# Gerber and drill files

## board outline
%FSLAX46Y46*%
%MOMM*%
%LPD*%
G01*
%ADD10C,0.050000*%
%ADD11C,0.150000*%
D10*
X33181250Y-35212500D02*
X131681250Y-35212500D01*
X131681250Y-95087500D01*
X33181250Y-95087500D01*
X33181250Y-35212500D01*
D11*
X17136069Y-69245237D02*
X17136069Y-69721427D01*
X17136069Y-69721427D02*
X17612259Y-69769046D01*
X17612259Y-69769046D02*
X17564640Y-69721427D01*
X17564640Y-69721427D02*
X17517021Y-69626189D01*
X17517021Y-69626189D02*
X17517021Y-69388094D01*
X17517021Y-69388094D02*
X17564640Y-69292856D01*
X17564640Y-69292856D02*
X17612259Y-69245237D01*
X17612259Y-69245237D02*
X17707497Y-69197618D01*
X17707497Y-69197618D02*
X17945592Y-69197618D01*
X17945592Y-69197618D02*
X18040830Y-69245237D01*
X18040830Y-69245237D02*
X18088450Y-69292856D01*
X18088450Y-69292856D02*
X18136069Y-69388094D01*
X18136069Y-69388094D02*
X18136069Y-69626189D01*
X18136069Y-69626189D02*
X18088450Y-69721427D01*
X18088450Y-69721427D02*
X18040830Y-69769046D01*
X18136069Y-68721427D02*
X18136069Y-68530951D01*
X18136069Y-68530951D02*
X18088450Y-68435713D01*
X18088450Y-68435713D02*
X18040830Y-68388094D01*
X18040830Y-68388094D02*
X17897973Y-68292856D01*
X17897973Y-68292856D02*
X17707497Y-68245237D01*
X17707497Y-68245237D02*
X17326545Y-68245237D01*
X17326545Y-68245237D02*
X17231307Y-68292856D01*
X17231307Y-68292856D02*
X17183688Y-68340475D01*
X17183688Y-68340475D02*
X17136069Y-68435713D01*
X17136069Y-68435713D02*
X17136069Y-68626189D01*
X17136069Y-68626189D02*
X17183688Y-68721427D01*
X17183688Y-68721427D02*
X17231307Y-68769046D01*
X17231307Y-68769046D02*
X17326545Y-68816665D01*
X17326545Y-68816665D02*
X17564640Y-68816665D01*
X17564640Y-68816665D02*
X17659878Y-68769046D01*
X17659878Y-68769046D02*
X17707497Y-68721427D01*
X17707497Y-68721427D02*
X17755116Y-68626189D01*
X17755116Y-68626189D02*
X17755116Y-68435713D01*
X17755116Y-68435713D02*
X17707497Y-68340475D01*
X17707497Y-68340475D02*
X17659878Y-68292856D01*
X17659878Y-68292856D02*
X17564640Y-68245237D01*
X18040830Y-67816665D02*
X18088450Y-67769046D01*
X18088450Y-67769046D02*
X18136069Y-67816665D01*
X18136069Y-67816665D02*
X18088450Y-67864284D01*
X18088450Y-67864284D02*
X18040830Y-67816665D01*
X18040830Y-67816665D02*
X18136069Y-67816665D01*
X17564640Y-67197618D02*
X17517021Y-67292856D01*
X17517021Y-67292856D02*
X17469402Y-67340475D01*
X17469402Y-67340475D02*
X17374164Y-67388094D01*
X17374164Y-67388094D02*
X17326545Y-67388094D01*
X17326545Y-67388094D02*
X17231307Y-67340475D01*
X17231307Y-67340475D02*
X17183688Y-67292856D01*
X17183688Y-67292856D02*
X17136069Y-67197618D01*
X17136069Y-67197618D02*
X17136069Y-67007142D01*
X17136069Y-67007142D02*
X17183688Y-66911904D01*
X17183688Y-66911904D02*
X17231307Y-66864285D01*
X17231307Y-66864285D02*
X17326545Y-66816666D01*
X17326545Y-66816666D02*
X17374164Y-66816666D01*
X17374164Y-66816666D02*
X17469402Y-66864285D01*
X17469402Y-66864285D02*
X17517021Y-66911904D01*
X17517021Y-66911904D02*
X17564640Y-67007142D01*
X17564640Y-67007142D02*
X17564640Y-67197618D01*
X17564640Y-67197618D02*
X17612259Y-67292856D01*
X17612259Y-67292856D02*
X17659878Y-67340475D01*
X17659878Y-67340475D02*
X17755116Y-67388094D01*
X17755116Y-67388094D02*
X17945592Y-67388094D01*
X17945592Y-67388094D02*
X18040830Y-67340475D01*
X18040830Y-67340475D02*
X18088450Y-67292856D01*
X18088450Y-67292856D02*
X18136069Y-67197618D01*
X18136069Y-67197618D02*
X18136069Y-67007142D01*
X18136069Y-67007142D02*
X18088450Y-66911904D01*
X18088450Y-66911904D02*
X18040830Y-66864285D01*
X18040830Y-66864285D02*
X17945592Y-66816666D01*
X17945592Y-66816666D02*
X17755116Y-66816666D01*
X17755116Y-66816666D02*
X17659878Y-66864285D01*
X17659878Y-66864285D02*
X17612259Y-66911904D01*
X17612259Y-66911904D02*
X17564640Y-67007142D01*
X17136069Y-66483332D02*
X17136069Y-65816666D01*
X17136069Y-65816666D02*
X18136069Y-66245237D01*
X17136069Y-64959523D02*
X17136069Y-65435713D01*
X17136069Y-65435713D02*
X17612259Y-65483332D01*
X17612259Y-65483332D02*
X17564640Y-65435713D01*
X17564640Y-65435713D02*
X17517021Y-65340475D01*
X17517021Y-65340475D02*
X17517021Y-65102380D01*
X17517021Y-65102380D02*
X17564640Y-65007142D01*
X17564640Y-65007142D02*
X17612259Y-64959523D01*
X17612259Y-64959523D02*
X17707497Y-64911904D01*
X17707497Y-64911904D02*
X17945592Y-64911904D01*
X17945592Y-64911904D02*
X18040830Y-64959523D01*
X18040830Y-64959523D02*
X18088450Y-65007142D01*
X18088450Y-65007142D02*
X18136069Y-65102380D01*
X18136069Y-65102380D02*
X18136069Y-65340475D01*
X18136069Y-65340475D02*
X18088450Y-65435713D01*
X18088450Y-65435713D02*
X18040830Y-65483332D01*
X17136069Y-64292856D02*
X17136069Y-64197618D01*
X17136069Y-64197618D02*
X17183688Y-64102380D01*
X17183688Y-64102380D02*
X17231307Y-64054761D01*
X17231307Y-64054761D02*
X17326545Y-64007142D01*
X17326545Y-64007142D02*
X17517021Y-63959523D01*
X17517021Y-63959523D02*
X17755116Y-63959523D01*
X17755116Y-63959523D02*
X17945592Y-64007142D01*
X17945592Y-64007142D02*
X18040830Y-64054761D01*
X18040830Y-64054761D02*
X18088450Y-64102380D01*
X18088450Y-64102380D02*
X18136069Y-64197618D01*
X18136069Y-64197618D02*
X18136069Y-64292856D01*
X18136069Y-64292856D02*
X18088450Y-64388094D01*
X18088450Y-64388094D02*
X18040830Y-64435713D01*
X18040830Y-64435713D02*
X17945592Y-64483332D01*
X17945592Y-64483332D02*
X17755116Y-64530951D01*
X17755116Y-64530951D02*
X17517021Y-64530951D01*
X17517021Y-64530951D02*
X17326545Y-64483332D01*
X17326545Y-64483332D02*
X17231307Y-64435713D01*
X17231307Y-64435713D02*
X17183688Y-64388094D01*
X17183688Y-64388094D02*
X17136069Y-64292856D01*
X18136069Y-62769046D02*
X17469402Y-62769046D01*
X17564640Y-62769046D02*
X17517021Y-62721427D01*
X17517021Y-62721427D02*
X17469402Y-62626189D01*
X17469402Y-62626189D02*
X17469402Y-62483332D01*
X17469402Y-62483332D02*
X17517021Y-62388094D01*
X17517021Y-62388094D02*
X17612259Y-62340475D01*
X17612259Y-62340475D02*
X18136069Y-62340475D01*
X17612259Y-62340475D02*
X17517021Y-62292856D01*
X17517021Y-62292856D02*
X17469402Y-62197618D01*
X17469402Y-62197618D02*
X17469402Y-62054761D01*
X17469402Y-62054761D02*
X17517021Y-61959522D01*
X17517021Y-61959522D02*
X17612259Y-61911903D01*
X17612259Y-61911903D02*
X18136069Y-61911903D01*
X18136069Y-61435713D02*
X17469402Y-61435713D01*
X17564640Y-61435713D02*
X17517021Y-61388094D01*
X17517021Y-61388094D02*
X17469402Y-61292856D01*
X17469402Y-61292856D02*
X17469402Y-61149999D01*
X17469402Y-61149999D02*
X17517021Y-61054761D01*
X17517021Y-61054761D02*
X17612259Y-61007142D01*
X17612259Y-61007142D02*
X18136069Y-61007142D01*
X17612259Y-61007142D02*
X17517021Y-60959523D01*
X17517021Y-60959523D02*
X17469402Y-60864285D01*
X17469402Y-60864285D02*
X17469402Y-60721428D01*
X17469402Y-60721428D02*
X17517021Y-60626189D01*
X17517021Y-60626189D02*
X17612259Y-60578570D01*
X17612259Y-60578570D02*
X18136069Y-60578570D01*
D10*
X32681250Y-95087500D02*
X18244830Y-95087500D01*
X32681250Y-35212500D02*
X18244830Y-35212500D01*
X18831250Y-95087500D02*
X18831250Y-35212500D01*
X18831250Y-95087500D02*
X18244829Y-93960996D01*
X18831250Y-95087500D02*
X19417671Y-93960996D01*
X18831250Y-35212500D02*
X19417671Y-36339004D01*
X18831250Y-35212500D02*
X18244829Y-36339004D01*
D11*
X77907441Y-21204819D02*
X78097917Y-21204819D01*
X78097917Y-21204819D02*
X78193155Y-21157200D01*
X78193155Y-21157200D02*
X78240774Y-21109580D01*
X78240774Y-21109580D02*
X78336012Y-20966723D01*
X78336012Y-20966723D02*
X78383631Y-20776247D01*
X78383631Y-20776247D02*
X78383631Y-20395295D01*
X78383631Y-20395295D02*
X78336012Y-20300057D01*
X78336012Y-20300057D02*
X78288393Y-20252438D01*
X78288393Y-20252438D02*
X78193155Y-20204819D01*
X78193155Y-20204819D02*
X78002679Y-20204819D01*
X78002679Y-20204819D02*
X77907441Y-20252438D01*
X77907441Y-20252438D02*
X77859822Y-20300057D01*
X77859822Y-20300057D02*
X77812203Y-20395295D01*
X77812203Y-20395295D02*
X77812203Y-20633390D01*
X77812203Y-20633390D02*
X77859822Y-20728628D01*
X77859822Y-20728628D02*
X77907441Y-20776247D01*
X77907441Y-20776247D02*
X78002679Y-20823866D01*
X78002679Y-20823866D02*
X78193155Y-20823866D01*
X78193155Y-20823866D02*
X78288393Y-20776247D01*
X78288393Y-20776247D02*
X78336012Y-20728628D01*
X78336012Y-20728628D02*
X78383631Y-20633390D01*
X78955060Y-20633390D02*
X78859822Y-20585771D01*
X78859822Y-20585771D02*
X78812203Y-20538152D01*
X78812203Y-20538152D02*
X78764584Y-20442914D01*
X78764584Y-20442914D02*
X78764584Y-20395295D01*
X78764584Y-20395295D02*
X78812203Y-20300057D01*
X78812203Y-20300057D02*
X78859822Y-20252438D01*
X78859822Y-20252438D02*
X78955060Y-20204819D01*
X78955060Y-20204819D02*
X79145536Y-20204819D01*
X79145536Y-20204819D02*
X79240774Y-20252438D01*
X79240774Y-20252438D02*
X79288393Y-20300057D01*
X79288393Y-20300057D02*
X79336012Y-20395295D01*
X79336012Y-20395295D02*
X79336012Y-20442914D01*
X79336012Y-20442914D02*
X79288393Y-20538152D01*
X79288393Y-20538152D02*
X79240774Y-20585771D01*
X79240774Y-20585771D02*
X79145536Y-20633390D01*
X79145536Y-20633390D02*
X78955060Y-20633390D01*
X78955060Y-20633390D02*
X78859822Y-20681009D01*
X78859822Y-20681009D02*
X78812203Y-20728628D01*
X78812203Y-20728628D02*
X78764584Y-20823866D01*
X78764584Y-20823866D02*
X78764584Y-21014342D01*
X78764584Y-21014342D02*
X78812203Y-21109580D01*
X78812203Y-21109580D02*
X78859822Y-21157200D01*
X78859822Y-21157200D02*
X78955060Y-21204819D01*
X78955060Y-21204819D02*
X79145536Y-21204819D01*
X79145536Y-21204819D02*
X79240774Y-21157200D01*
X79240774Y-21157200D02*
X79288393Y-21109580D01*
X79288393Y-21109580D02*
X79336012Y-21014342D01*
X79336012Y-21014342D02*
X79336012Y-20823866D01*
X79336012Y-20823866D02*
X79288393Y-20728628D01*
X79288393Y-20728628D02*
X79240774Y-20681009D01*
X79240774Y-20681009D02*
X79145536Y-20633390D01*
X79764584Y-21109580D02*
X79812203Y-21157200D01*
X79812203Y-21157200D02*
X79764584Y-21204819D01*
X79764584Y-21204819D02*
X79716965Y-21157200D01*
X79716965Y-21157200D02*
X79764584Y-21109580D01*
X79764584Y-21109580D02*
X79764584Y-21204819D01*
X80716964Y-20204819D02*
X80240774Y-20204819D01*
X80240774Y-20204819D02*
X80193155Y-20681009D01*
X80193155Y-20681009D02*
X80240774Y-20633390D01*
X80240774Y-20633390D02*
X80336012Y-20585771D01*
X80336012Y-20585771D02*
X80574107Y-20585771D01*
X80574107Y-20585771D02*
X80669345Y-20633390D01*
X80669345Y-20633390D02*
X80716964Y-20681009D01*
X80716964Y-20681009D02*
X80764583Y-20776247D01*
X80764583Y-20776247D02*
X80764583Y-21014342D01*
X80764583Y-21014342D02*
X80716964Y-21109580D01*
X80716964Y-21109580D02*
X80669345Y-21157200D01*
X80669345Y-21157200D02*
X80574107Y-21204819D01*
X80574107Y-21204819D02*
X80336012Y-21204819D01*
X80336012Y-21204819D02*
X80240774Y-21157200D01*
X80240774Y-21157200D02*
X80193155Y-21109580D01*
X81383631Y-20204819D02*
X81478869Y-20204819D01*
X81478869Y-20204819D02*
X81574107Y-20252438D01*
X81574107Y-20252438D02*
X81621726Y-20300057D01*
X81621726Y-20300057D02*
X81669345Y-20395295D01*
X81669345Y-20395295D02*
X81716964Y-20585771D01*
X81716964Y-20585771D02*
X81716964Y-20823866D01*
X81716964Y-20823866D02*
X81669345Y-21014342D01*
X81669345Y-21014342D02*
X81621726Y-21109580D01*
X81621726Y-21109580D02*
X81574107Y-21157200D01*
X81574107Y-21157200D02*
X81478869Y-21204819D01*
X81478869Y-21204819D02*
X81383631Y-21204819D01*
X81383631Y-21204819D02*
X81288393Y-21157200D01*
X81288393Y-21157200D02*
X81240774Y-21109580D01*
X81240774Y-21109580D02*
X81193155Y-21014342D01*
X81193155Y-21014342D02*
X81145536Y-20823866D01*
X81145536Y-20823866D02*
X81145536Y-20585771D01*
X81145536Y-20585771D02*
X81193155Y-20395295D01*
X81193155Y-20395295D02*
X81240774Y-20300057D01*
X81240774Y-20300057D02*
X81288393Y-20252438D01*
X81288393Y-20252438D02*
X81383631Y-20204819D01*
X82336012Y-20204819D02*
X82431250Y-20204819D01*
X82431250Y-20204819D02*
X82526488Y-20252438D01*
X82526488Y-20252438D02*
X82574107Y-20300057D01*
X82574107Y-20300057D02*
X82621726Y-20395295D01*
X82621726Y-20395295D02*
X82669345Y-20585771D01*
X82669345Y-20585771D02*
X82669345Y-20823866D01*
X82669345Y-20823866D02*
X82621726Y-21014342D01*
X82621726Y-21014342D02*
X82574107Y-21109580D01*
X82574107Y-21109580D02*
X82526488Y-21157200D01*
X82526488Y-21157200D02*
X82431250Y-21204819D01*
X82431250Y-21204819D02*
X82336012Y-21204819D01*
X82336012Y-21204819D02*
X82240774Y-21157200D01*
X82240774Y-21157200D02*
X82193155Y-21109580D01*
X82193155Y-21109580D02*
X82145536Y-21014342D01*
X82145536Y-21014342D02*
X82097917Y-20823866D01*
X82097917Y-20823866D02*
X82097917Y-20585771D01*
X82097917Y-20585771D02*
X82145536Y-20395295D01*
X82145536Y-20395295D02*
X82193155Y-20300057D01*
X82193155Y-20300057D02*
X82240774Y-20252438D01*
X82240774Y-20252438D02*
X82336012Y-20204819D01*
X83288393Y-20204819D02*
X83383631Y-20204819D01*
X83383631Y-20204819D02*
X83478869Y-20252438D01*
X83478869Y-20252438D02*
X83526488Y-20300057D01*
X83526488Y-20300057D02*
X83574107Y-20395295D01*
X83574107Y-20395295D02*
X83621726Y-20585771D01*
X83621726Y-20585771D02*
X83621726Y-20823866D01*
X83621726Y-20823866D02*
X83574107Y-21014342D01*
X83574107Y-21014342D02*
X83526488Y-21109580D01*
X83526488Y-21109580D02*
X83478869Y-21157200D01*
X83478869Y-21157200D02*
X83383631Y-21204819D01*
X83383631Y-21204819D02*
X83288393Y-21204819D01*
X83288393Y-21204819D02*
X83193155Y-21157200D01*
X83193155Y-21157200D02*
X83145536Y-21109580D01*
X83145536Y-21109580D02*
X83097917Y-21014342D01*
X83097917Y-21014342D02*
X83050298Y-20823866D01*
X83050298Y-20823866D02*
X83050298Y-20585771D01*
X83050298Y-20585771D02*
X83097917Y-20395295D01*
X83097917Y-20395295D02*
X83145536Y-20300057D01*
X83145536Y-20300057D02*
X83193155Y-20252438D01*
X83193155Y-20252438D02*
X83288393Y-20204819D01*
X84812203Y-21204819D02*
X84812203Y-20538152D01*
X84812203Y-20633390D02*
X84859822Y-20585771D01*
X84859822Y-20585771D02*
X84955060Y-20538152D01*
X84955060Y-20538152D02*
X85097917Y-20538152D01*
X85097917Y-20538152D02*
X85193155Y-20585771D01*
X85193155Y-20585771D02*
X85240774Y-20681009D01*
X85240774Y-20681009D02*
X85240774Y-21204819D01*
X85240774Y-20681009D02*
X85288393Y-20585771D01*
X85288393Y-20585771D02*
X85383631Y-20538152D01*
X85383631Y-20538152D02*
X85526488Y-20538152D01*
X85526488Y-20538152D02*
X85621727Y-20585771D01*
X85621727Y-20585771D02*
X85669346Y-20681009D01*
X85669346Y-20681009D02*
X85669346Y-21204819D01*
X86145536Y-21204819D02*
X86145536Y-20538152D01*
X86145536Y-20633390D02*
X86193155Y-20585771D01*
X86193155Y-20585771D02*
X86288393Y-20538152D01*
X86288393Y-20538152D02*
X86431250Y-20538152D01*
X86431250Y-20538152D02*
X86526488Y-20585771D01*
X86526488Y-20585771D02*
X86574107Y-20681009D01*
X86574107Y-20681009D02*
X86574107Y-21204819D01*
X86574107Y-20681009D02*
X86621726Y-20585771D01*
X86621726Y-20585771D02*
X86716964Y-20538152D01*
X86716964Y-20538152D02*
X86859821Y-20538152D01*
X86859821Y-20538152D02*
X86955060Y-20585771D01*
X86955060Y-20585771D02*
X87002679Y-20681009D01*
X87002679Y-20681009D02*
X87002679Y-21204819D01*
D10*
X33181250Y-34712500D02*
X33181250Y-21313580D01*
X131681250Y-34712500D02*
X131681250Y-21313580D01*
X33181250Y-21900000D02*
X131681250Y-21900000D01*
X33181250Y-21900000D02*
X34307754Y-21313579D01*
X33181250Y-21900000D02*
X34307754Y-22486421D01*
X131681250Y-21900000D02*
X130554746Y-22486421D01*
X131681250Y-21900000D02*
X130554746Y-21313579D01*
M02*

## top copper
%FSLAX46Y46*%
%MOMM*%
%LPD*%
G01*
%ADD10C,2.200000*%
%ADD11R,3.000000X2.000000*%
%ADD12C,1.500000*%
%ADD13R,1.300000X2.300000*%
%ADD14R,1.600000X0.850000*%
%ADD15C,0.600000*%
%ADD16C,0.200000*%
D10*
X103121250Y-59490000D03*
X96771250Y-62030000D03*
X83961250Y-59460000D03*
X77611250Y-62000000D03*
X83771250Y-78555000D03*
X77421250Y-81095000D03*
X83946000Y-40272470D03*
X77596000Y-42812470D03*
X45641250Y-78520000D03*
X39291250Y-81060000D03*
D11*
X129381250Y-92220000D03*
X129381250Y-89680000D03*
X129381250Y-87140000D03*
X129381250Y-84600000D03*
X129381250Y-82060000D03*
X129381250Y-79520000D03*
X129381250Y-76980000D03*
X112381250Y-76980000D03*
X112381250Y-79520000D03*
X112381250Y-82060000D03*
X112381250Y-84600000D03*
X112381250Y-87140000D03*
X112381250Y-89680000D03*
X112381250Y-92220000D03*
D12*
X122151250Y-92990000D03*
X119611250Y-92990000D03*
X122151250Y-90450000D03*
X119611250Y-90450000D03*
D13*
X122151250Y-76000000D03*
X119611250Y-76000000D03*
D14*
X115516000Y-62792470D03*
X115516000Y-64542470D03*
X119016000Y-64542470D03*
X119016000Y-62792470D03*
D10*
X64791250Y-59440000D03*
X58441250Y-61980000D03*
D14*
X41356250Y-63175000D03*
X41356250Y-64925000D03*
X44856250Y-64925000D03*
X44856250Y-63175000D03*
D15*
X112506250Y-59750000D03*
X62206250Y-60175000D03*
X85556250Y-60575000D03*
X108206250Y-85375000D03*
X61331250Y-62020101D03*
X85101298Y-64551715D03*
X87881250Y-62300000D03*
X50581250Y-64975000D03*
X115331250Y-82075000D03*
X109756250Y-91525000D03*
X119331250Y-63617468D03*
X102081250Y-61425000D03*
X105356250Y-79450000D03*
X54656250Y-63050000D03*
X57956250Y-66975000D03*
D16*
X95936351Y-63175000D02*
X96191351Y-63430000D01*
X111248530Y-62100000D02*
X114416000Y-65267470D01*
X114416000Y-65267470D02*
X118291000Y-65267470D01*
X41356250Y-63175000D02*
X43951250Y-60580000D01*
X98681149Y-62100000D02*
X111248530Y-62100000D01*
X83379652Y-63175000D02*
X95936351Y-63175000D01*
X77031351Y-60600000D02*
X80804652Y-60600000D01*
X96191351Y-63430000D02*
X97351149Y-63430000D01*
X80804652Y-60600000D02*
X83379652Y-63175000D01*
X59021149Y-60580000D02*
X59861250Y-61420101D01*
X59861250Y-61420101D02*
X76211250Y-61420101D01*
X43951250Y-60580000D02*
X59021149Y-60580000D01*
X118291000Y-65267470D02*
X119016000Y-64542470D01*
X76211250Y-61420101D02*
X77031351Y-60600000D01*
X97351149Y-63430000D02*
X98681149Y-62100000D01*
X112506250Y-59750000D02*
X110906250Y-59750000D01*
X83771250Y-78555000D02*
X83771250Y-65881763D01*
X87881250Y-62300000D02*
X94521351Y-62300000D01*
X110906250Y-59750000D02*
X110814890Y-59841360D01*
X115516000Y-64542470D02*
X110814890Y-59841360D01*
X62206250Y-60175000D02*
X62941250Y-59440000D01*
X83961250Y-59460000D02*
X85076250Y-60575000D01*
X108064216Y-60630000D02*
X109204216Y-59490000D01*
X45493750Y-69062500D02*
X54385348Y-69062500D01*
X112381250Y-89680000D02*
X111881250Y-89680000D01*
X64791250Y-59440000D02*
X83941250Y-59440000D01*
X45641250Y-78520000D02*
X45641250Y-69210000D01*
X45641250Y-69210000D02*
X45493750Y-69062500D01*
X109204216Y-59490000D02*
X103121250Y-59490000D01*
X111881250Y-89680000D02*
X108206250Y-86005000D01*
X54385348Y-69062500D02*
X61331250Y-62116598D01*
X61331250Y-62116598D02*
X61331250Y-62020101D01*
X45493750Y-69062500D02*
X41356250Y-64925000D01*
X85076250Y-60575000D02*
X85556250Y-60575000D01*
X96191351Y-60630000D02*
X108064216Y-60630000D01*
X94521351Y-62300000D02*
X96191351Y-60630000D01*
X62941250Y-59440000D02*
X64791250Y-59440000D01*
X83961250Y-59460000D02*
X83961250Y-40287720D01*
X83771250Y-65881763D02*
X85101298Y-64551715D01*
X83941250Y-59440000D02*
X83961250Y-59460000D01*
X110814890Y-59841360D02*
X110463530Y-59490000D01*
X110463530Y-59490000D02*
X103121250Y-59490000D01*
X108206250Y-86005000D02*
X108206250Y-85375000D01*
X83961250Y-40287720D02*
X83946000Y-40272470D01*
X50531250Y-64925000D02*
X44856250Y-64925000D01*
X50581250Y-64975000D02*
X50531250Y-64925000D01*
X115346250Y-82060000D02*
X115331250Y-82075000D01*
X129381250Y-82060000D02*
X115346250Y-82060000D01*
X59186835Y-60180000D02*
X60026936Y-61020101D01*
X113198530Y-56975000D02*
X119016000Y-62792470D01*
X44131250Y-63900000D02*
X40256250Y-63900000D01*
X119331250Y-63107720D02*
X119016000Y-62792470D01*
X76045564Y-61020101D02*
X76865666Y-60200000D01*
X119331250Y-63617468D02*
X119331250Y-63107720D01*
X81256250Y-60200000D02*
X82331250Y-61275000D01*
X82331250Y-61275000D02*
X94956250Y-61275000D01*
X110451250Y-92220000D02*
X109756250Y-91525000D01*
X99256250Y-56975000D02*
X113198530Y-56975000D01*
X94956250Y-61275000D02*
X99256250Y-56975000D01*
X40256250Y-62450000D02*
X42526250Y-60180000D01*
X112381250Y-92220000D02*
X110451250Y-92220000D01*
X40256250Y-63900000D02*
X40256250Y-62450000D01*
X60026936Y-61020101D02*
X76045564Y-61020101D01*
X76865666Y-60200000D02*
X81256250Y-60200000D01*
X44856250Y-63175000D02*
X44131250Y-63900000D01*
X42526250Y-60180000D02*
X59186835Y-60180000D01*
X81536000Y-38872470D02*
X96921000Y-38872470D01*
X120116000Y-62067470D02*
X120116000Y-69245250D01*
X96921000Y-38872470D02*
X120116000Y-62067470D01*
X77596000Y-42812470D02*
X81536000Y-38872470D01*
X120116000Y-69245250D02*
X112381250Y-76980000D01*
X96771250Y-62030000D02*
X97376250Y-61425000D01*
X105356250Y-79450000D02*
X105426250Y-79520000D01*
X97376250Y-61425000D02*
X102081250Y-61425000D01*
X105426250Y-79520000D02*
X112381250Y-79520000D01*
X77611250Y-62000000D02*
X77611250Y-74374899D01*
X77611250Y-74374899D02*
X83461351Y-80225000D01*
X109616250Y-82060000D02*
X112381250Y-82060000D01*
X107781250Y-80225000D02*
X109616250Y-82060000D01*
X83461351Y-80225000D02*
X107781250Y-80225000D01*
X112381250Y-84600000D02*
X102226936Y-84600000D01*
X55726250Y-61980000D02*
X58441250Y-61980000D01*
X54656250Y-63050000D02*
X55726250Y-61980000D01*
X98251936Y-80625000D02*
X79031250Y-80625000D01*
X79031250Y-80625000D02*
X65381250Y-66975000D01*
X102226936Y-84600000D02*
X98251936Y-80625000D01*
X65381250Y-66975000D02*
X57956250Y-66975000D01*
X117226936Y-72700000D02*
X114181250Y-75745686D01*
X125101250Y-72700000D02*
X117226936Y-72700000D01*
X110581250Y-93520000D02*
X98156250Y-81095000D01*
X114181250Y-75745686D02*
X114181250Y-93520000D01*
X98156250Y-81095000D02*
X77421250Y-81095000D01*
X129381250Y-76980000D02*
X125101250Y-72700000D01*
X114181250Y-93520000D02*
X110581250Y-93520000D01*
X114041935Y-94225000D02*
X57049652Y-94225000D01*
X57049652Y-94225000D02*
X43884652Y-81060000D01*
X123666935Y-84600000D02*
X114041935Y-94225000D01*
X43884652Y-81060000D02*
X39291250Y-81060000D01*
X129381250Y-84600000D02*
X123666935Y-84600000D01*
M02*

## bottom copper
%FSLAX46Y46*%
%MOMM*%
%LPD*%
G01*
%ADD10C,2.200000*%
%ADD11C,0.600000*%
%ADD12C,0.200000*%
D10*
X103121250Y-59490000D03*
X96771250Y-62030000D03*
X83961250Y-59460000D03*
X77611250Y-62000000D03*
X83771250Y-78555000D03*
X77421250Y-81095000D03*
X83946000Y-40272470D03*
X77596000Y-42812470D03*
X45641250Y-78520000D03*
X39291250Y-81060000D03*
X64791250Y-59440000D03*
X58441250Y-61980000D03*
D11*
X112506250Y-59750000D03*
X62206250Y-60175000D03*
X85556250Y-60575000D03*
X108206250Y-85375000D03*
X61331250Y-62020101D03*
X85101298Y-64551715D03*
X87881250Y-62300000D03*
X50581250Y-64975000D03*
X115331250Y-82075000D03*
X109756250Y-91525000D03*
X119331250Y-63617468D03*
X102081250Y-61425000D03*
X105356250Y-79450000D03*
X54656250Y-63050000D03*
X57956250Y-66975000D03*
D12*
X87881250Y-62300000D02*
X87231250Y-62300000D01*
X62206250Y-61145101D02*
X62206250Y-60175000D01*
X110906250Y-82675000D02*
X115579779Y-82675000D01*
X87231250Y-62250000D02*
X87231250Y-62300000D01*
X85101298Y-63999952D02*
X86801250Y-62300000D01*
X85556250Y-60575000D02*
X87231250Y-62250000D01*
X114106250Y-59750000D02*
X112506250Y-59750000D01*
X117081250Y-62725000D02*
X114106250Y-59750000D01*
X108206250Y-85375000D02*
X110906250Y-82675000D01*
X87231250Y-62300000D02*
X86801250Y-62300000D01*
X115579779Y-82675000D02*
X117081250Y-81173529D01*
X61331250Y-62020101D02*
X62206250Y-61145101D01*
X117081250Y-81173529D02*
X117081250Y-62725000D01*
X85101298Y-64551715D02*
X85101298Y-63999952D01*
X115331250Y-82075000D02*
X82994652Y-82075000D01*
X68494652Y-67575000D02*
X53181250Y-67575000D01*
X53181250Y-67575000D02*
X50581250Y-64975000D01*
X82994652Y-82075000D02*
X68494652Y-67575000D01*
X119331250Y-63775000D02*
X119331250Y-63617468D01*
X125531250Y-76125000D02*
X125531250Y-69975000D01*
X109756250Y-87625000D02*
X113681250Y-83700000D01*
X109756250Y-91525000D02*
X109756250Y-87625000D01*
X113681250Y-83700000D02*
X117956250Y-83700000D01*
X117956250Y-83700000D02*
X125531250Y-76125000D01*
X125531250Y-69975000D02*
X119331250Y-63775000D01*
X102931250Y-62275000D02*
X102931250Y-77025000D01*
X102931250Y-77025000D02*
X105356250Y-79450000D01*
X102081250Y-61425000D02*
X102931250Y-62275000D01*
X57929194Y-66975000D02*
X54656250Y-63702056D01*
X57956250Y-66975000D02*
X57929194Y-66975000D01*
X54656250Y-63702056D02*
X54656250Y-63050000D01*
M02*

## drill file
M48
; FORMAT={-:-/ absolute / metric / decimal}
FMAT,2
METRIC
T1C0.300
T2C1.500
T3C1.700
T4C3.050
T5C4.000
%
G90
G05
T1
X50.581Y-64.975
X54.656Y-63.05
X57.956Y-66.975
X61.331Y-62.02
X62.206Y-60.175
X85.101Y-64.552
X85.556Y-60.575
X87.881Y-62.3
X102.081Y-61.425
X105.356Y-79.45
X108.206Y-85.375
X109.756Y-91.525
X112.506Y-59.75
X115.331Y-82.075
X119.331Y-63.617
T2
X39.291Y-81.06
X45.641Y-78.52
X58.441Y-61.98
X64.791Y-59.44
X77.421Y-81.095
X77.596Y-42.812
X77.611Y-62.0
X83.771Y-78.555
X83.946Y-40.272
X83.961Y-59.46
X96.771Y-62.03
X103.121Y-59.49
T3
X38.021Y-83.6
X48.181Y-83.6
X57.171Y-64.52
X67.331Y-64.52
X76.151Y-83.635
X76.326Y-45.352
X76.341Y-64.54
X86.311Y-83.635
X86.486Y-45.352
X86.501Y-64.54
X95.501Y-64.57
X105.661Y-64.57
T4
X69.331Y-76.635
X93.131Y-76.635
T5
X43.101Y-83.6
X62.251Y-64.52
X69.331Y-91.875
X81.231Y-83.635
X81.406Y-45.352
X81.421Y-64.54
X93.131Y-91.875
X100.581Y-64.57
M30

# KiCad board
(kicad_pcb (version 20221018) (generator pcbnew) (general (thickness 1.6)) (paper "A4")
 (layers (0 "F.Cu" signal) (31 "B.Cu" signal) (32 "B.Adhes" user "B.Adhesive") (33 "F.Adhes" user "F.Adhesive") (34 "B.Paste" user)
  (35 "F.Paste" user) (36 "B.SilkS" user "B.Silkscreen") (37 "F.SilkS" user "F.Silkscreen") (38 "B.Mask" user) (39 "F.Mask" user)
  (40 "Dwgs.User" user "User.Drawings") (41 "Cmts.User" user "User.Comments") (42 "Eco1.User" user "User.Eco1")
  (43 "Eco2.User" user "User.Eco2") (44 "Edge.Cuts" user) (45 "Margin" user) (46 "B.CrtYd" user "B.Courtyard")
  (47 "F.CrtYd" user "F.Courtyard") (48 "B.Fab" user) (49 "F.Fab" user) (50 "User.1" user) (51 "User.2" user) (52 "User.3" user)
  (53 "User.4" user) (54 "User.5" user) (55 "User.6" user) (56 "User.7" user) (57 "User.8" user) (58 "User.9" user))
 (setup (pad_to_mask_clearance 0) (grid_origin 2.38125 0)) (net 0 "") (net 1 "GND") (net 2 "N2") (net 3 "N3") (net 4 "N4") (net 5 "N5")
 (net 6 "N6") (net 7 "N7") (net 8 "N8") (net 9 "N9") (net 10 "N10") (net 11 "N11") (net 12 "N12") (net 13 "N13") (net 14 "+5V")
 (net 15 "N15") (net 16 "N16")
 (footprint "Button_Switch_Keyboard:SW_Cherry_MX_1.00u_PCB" (layer "F.Cu") (at 103.12125 59.49)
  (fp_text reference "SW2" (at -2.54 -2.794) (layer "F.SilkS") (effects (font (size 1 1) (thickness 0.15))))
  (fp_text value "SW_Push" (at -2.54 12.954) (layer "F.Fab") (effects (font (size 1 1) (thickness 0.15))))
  (pad "" np_thru_hole circle (at -7.62 5.08) (size 1.7 1.7) (drill 1.7) (layers "*.Cu" "*.Mask"))
  (pad "" np_thru_hole circle (at -2.54 5.08) (size 4 4) (drill 4) (layers "*.Cu" "*.Mask"))
  (pad "" np_thru_hole circle (at 2.54 5.08) (size 1.7 1.7) (drill 1.7) (layers "*.Cu" "*.Mask"))
  (pad "1" thru_hole circle (at 0 0) (size 2.2 2.2) (drill 1.5) (layers "*.Cu" "*.Mask") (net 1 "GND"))
  (pad "2" thru_hole circle (at -6.35 2.54) (size 2.2 2.2) (drill 1.5) (layers "*.Cu" "*.Mask") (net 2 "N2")))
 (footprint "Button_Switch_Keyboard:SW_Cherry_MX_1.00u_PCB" (layer "F.Cu") (at 83.96125 59.46)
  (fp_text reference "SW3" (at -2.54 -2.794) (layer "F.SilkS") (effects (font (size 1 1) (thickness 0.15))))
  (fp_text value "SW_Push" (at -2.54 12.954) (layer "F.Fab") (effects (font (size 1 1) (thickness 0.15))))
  (pad "" np_thru_hole circle (at -7.62 5.08) (size 1.7 1.7) (drill 1.7) (layers "*.Cu" "*.Mask"))
  (pad "" np_thru_hole circle (at -2.54 5.08) (size 4 4) (drill 4) (layers "*.Cu" "*.Mask"))
  (pad "" np_thru_hole circle (at 2.54 5.08) (size 1.7 1.7) (drill 1.7) (layers "*.Cu" "*.Mask"))
  (pad "1" thru_hole circle (at 0 0) (size 2.2 2.2) (drill 1.5) (layers "*.Cu" "*.Mask") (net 1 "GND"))
  (pad "2" thru_hole circle (at -6.35 2.54) (size 2.2 2.2) (drill 1.5) (layers "*.Cu" "*.Mask") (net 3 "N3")))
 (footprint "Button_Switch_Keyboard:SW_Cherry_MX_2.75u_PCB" (layer "F.Cu") (at 83.77125 78.555)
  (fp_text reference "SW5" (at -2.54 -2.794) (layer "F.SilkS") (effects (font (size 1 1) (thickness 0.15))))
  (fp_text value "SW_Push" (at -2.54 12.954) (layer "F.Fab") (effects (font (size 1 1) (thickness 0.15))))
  (pad "" np_thru_hole circle (at -14.44 -1.92) (size 3.05 3.05) (drill 3.05) (layers "*.Cu" "*.Mask"))
  (pad "" np_thru_hole circle (at -14.44 13.32) (size 4 4) (drill 4) (layers "*.Cu" "*.Mask"))
  (pad "" np_thru_hole circle (at -7.62 5.08) (size 1.7 1.7) (drill 1.7) (layers "*.Cu" "*.Mask"))
  (pad "" np_thru_hole circle (at -2.54 5.08) (size 4 4) (drill 4) (layers "*.Cu" "*.Mask"))
  (pad "" np_thru_hole circle (at 2.54 5.08) (size 1.7 1.7) (drill 1.7) (layers "*.Cu" "*.Mask"))
  (pad "" np_thru_hole circle (at 9.36 -1.92) (size 3.05 3.05) (drill 3.05) (layers "*.Cu" "*.Mask"))
  (pad "" np_thru_hole circle (at 9.36 13.32) (size 4 4) (drill 4) (layers "*.Cu" "*.Mask"))
  (pad "1" thru_hole circle (at 0 0) (size 2.2 2.2) (drill 1.5) (layers "*.Cu" "*.Mask") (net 1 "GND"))
  (pad "2" thru_hole circle (at -6.35 2.54) (size 2.2 2.2) (drill 1.5) (layers "*.Cu" "*.Mask") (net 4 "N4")))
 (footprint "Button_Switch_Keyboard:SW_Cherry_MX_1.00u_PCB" (layer "F.Cu") (at 83.946 40.27247)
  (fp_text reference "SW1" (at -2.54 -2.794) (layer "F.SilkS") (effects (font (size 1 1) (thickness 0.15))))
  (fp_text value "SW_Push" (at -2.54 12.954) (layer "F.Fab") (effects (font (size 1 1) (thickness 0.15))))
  (pad "" np_thru_hole circle (at -7.62 5.08) (size 1.7 1.7) (drill 1.7) (layers "*.Cu" "*.Mask"))
  (pad "" np_thru_hole circle (at -2.54 5.08) (size 4 4) (drill 4) (layers "*.Cu" "*.Mask"))
  (pad "" np_thru_hole circle (at 2.54 5.08) (size 1.7 1.7) (drill 1.7) (layers "*.Cu" "*.Mask"))
  (pad "1" thru_hole circle (at 0 0) (size 2.2 2.2) (drill 1.5) (layers "*.Cu" "*.Mask") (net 1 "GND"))
  (pad "2" thru_hole circle (at -6.35 2.54) (size 2.2 2.2) (drill 1.5) (layers "*.Cu" "*.Mask") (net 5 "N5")))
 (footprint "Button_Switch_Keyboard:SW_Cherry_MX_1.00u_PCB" (layer "F.Cu") (at 45.64125 78.52)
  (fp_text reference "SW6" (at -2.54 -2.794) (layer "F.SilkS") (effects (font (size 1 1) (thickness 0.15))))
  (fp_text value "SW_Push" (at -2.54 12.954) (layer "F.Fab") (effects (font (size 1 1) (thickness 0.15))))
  (pad "" np_thru_hole circle (at -7.62 5.08) (size 1.7 1.7) (drill 1.7) (layers "*.Cu" "*.Mask"))
  (pad "" np_thru_hole circle (at -2.54 5.08) (size 4 4) (drill 4) (layers "*.Cu" "*.Mask"))
  (pad "" np_thru_hole circle (at 2.54 5.08) (size 1.7 1.7) (drill 1.7) (layers "*.Cu" "*.Mask"))
  (pad "1" thru_hole circle (at 0 0) (size 2.2 2.2) (drill 1.5) (layers "*.Cu" "*.Mask") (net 1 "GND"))
  (pad "2" thru_hole circle (at -6.35 2.54) (size 2.2 2.2) (drill 1.5) (layers "*.Cu" "*.Mask") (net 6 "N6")))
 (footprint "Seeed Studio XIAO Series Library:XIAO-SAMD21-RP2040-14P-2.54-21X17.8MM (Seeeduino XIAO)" (layer "F.Cu") (at 120.88125 84.6 180)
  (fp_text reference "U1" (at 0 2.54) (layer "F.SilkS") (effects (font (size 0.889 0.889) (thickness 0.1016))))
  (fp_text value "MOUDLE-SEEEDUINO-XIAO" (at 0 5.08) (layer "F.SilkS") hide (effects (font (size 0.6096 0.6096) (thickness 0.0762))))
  (pad "1" smd rect (at -8.5 -7.62 180) (size 3 2) (layers "F.Cu" "F.Paste" "F.Mask") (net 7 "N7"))
  (pad "2" smd rect (at -8.5 -5.08 180) (size 3 2) (layers "F.Cu" "F.Paste" "F.Mask") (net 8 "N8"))
  (pad "3" smd rect (at -8.5 -2.54 180) (size 3 2) (layers "F.Cu" "F.Paste" "F.Mask") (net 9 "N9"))
  (pad "4" smd rect (at -8.5 0 180) (size 3 2) (layers "F.Cu" "F.Paste" "F.Mask") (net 6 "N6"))
  (pad "5" smd rect (at -8.5 2.54 180) (size 3 2) (layers "F.Cu" "F.Paste" "F.Mask") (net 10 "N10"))
  (pad "6" smd rect (at -8.5 5.08) (size 3 2) (layers "F.Cu" "F.Paste" "F.Mask") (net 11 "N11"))
  (pad "7" smd rect (at -8.5 7.62 180) (size 3 2) (layers "F.Cu" "F.Paste" "F.Mask") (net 4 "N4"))
  (pad "8" smd rect (at 8.5 7.62 180) (size 3 2) (layers "F.Cu" "F.Paste" "F.Mask") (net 5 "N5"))
  (pad "9" smd rect (at 8.5 5.08 180) (size 3 2) (layers "F.Cu" "F.Paste" "F.Mask") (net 2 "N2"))
  (pad "10" smd rect (at 8.5 2.54 180) (size 3 2) (layers "F.Cu" "F.Paste" "F.Mask") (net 3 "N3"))
  (pad "11" smd rect (at 8.5 0 180) (size 3 2) (layers "F.Cu" "F.Paste" "F.Mask") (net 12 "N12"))
  (pad "12" smd rect (at 8.5 -2.54 180) (size 3 2) (layers "F.Cu" "F.Paste" "F.Mask") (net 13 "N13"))
  (pad "13" smd rect (at 8.5 -5.08 180) (size 3 2) (layers "F.Cu" "F.Paste" "F.Mask") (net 1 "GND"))
  (pad "14" smd rect (at 8.5 -7.62 180) (size 3 2) (layers "F.Cu" "F.Paste" "F.Mask") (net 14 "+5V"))
  (pad "15" smd circle (at -1.27 -8.39 270) (size 1.5 1.5) (layers "F.Cu" "F.Paste" "F.Mask"))
  (pad "16" smd circle (at 1.27 -8.39 270) (size 1.5 1.5) (layers "F.Cu" "F.Paste" "F.Mask"))
  (pad "17" smd circle (at -1.27 -5.85 270) (size 1.5 1.5) (layers "F.Cu" "F.Paste" "F.Mask"))
  (pad "18" smd circle (at 1.27 -5.85 270) (size 1.5 1.5) (layers "F.Cu" "F.Paste" "F.Mask"))
  (pad "19" smd rect (at -1.27 8.6 270) (size 2.3 1.3) (layers "F.Cu" "F.Paste" "F.Mask"))
  (pad "20" smd rect (at 1.27 8.6 270) (size 2.3 1.3) (layers "F.Cu" "F.Paste" "F.Mask")))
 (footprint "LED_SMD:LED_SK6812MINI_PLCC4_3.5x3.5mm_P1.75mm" (layer "F.Cu") (at 117.266 63.66747)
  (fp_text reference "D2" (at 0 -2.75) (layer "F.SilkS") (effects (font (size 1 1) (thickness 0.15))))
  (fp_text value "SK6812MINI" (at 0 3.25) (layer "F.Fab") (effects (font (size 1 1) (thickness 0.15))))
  (pad "1" smd rect (at -1.75 -0.875) (size 1.6 0.85) (layers "F.Cu" "F.Paste" "F.Mask") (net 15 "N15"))
  (pad "2" smd rect (at -1.75 0.875) (size 1.6 0.85) (layers "F.Cu" "F.Paste" "F.Mask") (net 1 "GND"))
  (pad "3" smd rect (at 1.75 0.875) (size 1.6 0.85) (layers "F.Cu" "F.Paste" "F.Mask") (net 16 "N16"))
  (pad "4" smd rect (at 1.75 -0.875) (size 1.6 0.85) (layers "F.Cu" "F.Paste" "F.Mask") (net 14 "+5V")))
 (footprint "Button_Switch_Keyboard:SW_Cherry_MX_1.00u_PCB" (layer "F.Cu") (at 64.79125 59.44)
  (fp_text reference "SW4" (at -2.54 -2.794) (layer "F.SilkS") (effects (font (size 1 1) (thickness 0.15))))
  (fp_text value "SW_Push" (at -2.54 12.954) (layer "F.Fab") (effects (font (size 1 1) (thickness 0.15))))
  (pad "" np_thru_hole circle (at -7.62 5.08) (size 1.7 1.7) (drill 1.7) (layers "*.Cu" "*.Mask"))
  (pad "" np_thru_hole circle (at -2.54 5.08) (size 4 4) (drill 4) (layers "*.Cu" "*.Mask"))
  (pad "" np_thru_hole circle (at 2.54 5.08) (size 1.7 1.7) (drill 1.7) (layers "*.Cu" "*.Mask"))
  (pad "1" thru_hole circle (at 0 0) (size 2.2 2.2) (drill 1.5) (layers "*.Cu" "*.Mask") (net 1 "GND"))
  (pad "2" thru_hole circle (at -6.35 2.54) (size 2.2 2.2) (drill 1.5) (layers "*.Cu" "*.Mask") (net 12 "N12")))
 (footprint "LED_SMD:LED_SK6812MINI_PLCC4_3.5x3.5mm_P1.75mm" (layer "F.Cu") (at 43.10625 64.05)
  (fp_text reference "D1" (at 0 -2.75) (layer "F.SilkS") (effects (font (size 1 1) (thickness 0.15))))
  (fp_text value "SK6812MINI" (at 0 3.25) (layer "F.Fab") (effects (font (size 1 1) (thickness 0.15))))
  (pad "1" smd rect (at -1.75 -0.875) (size 1.6 0.85) (layers "F.Cu" "F.Paste" "F.Mask") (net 16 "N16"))
  (pad "2" smd rect (at -1.75 0.875) (size 1.6 0.85) (layers "F.Cu" "F.Paste" "F.Mask") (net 1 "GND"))
  (pad "3" smd rect (at 1.75 0.875) (size 1.6 0.85) (layers "F.Cu" "F.Paste" "F.Mask") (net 10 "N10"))
  (pad "4" smd rect (at 1.75 -0.875) (size 1.6 0.85) (layers "F.Cu" "F.Paste" "F.Mask") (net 14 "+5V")))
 (gr_rect (start 33.18125 35.2125) (end 131.68125 95.0875) (stroke (width 0.05) (type default)) (fill none) (layer "Edge.Cuts"))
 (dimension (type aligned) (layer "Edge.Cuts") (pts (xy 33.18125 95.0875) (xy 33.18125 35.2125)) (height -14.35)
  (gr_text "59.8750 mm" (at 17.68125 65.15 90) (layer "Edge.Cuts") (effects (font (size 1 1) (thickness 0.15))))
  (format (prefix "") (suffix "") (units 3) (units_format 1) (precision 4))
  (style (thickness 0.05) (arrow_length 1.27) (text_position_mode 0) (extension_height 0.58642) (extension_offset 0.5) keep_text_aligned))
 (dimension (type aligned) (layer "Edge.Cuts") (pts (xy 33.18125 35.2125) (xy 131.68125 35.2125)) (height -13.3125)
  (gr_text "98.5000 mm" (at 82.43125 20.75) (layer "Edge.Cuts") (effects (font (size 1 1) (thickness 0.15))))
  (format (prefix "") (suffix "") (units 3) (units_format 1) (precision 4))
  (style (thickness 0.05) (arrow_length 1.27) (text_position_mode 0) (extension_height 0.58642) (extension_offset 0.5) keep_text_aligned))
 (segment (start 95.936351 63.175) (end 96.191351 63.43) (width 0.2) (layer "F.Cu") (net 16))
 (segment (start 111.24853 62.1) (end 114.416 65.26747) (width 0.2) (layer "F.Cu") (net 16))
 (segment (start 114.416 65.26747) (end 118.291 65.26747) (width 0.2) (layer "F.Cu") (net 16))
 (segment (start 41.35625 63.175) (end 43.95125 60.58) (width 0.2) (layer "F.Cu") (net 16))
 (segment (start 98.681149 62.1) (end 111.24853 62.1) (width 0.2) (layer "F.Cu") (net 16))
 (segment (start 83.379652 63.175) (end 95.936351 63.175) (width 0.2) (layer "F.Cu") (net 16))
 (segment (start 77.031351 60.6) (end 80.804652 60.6) (width 0.2) (layer "F.Cu") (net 16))
 (segment (start 96.191351 63.43) (end 97.351149 63.43) (width 0.2) (layer "F.Cu") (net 16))
 (segment (start 80.804652 60.6) (end 83.379652 63.175) (width 0.2) (layer "F.Cu") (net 16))
 (segment (start 59.021149 60.58) (end 59.86125 61.420101) (width 0.2) (layer "F.Cu") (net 16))
 (segment (start 59.86125 61.420101) (end 76.21125 61.420101) (width 0.2) (layer "F.Cu") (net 16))
 (segment (start 43.95125 60.58) (end 59.021149 60.58) (width 0.2) (layer "F.Cu") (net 16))
 (segment (start 118.291 65.26747) (end 119.016 64.54247) (width 0.2) (layer "F.Cu") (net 16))
 (segment (start 76.21125 61.420101) (end 77.031351 60.6) (width 0.2) (layer "F.Cu") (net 16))
 (segment (start 97.351149 63.43) (end 98.681149 62.1) (width 0.2) (layer "F.Cu") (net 16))
 (segment (start 112.50625 59.75) (end 110.90625 59.75) (width 0.2) (layer "F.Cu") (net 1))
 (segment (start 83.77125 78.555) (end 83.77125 65.881763) (width 0.2) (layer "F.Cu") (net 1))
 (segment (start 87.88125 62.3) (end 94.521351 62.3) (width 0.2) (layer "F.Cu") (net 1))
 (segment (start 110.90625 59.75) (end 110.81489 59.84136) (width 0.2) (layer "F.Cu") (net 1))
 (segment (start 115.516 64.54247) (end 110.81489 59.84136) (width 0.2) (layer "F.Cu") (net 1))
 (segment (start 62.20625 60.175) (end 62.94125 59.44) (width 0.2) (layer "F.Cu") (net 1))
 (segment (start 83.96125 59.46) (end 85.07625 60.575) (width 0.2) (layer "F.Cu") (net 1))
 (segment (start 108.064216 60.63) (end 109.204216 59.49) (width 0.2) (layer "F.Cu") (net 1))
 (segment (start 45.49375 69.0625) (end 54.385348 69.0625) (width 0.2) (layer "F.Cu") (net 1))
 (segment (start 112.38125 89.68) (end 111.88125 89.68) (width 0.2) (layer "F.Cu") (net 1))
 (segment (start 64.79125 59.44) (end 83.94125 59.44) (width 0.2) (layer "F.Cu") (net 1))
 (segment (start 45.64125 78.52) (end 45.64125 69.21) (width 0.2) (layer "F.Cu") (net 1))
 (segment (start 45.64125 69.21) (end 45.49375 69.0625) (width 0.2) (layer "F.Cu") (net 1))
 (segment (start 109.204216 59.49) (end 103.12125 59.49) (width 0.2) (layer "F.Cu") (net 1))
 (segment (start 111.88125 89.68) (end 108.20625 86.005) (width 0.2) (layer "F.Cu") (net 1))
 (segment (start 54.385348 69.0625) (end 61.33125 62.116598) (width 0.2) (layer "F.Cu") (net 1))
 (segment (start 61.33125 62.116598) (end 61.33125 62.020101) (width 0.2) (layer "F.Cu") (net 1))
 (segment (start 45.49375 69.0625) (end 41.35625 64.925) (width 0.2) (layer "F.Cu") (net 1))
 (segment (start 85.07625 60.575) (end 85.55625 60.575) (width 0.2) (layer "F.Cu") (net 1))
 (segment (start 96.191351 60.63) (end 108.064216 60.63) (width 0.2) (layer "F.Cu") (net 1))
 (segment (start 94.521351 62.3) (end 96.191351 60.63) (width 0.2) (layer "F.Cu") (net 1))
 (segment (start 62.94125 59.44) (end 64.79125 59.44) (width 0.2) (layer "F.Cu") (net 1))
 (segment (start 83.96125 59.46) (end 83.96125 40.28772) (width 0.2) (layer "F.Cu") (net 1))
 (segment (start 83.77125 65.881763) (end 85.101298 64.551715) (width 0.2) (layer "F.Cu") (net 1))
 (segment (start 83.94125 59.44) (end 83.96125 59.46) (width 0.2) (layer "F.Cu") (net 1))
 (segment (start 110.81489 59.84136) (end 110.46353 59.49) (width 0.2) (layer "F.Cu") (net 1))
 (segment (start 110.46353 59.49) (end 103.12125 59.49) (width 0.2) (layer "F.Cu") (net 1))
 (segment (start 108.20625 86.005) (end 108.20625 85.375) (width 0.2) (layer "F.Cu") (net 1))
 (segment (start 83.96125 40.28772) (end 83.946 40.27247) (width 0.2) (layer "F.Cu") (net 1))
 (via (at 112.50625 59.75) (size 0.6) (drill 0.3) (layers "F.Cu" "B.Cu") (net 1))
 (via (at 62.20625 60.175) (size 0.6) (drill 0.3) (layers "F.Cu" "B.Cu") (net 1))
 (via (at 85.55625 60.575) (size 0.6) (drill 0.3) (layers "F.Cu" "B.Cu") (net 1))
 (via (at 108.20625 85.375) (size 0.6) (drill 0.3) (layers "F.Cu" "B.Cu") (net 1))
 (via (at 61.33125 62.020101) (size 0.6) (drill 0.3) (layers "F.Cu" "B.Cu") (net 1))
 (via (at 85.101298 64.551715) (size 0.6) (drill 0.3) (layers "F.Cu" "B.Cu") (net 1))
 (via (at 87.88125 62.3) (size 0.6) (drill 0.3) (layers "F.Cu" "B.Cu") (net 1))
 (segment (start 87.88125 62.3) (end 87.23125 62.3) (width 0.2) (layer "B.Cu") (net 1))
 (segment (start 62.20625 61.145101) (end 62.20625 60.175) (width 0.2) (layer "B.Cu") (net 1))
 (segment (start 110.90625 82.675) (end 115.579779 82.675) (width 0.2) (layer "B.Cu") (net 1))
 (segment (start 87.23125 62.25) (end 87.23125 62.3) (width 0.2) (layer "B.Cu") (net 1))
 (segment (start 85.101298 63.999952) (end 86.80125 62.3) (width 0.2) (layer "B.Cu") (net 1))
 (segment (start 85.55625 60.575) (end 87.23125 62.25) (width 0.2) (layer "B.Cu") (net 1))
 (segment (start 114.10625 59.75) (end 112.50625 59.75) (width 0.2) (layer "B.Cu") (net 1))
 (segment (start 117.08125 62.725) (end 114.10625 59.75) (width 0.2) (layer "B.Cu") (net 1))
 (segment (start 108.20625 85.375) (end 110.90625 82.675) (width 0.2) (layer "B.Cu") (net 1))
 (segment (start 87.23125 62.3) (end 86.80125 62.3) (width 0.2) (layer "B.Cu") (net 1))
 (segment (start 115.579779 82.675) (end 117.08125 81.173529) (width 0.2) (layer "B.Cu") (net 1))
 (segment (start 61.33125 62.020101) (end 62.20625 61.145101) (width 0.2) (layer "B.Cu") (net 1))
 (segment (start 117.08125 81.173529) (end 117.08125 62.725) (width 0.2) (layer "B.Cu") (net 1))
 (segment (start 85.101298 64.551715) (end 85.101298 63.999952) (width 0.2) (layer "B.Cu") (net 1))
 (segment (start 50.53125 64.925) (end 44.85625 64.925) (width 0.2) (layer "F.Cu") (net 10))
 (segment (start 50.58125 64.975) (end 50.53125 64.925) (width 0.2) (layer "F.Cu") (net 10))
 (segment (start 115.34625 82.06) (end 115.33125 82.075) (width 0.2) (layer "F.Cu") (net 10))
 (segment (start 129.38125 82.06) (end 115.34625 82.06) (width 0.2) (layer "F.Cu") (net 10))
 (via (at 50.58125 64.975) (size 0.6) (drill 0.3) (layers "F.Cu" "B.Cu") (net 10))
 (via (at 115.33125 82.075) (size 0.6) (drill 0.3) (layers "F.Cu" "B.Cu") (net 10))
 (segment (start 115.33125 82.075) (end 82.994652 82.075) (width 0.2) (layer "B.Cu") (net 10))
 (segment (start 68.494652 67.575) (end 53.18125 67.575) (width 0.2) (layer "B.Cu") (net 10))
 (segment (start 53.18125 67.575) (end 50.58125 64.975) (width 0.2) (layer "B.Cu") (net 10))
 (segment (start 82.994652 82.075) (end 68.494652 67.575) (width 0.2) (layer "B.Cu") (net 10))
 (segment (start 59.186835 60.18) (end 60.026936 61.020101) (width 0.2) (layer "F.Cu") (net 14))
 (segment (start 113.19853 56.975) (end 119.016 62.79247) (width 0.2) (layer "F.Cu") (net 14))
 (segment (start 44.13125 63.9) (end 40.25625 63.9) (width 0.2) (layer "F.Cu") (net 14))
 (segment (start 119.33125 63.10772) (end 119.016 62.79247) (width 0.2) (layer "F.Cu") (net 14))
 (segment (start 76.045564 61.020101) (end 76.865666 60.2) (width 0.2) (layer "F.Cu") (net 14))
 (segment (start 119.33125 63.617468) (end 119.33125 63.10772) (width 0.2) (layer "F.Cu") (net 14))
 (segment (start 81.25625 60.2) (end 82.33125 61.275) (width 0.2) (layer "F.Cu") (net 14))
 (segment (start 82.33125 61.275) (end 94.95625 61.275) (width 0.2) (layer "F.Cu") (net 14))
 (segment (start 110.45125 92.22) (end 109.75625 91.525) (width 0.2) (layer "F.Cu") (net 14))
 (segment (start 99.25625 56.975) (end 113.19853 56.975) (width 0.2) (layer "F.Cu") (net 14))
 (segment (start 94.95625 61.275) (end 99.25625 56.975) (width 0.2) (layer "F.Cu") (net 14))
 (segment (start 40.25625 62.45) (end 42.52625 60.18) (width 0.2) (layer "F.Cu") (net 14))
 (segment (start 112.38125 92.22) (end 110.45125 92.22) (width 0.2) (layer "F.Cu") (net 14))
 (segment (start 40.25625 63.9) (end 40.25625 62.45) (width 0.2) (layer "F.Cu") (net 14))
 (segment (start 60.026936 61.020101) (end 76.045564 61.020101) (width 0.2) (layer "F.Cu") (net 14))
 (segment (start 76.865666 60.2) (end 81.25625 60.2) (width 0.2) (layer "F.Cu") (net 14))
 (segment (start 44.85625 63.175) (end 44.13125 63.9) (width 0.2) (layer "F.Cu") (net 14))
 (segment (start 42.52625 60.18) (end 59.186835 60.18) (width 0.2) (layer "F.Cu") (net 14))
 (via (at 109.75625 91.525) (size 0.6) (drill 0.3) (layers "F.Cu" "B.Cu") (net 14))
 (via (at 119.33125 63.617468) (size 0.6) (drill 0.3) (layers "F.Cu" "B.Cu") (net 14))
 (segment (start 119.33125 63.775) (end 119.33125 63.617468) (width 0.2) (layer "B.Cu") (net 14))
 (segment (start 125.53125 76.125) (end 125.53125 69.975) (width 0.2) (layer "B.Cu") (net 14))
 (segment (start 109.75625 87.625) (end 113.68125 83.7) (width 0.2) (layer "B.Cu") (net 14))
 (segment (start 109.75625 91.525) (end 109.75625 87.625) (width 0.2) (layer "B.Cu") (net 14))
 (segment (start 113.68125 83.7) (end 117.95625 83.7) (width 0.2) (layer "B.Cu") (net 14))
 (segment (start 117.95625 83.7) (end 125.53125 76.125) (width 0.2) (layer "B.Cu") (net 14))
 (segment (start 125.53125 69.975) (end 119.33125 63.775) (width 0.2) (layer "B.Cu") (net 14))
 (segment (start 81.536 38.87247) (end 96.921 38.87247) (width 0.2) (layer "F.Cu") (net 5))
 (segment (start 120.116 62.06747) (end 120.116 69.24525) (width 0.2) (layer "F.Cu") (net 5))
 (segment (start 96.921 38.87247) (end 120.116 62.06747) (width 0.2) (layer "F.Cu") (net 5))
 (segment (start 77.596 42.81247) (end 81.536 38.87247) (width 0.2) (layer "F.Cu") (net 5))
 (segment (start 120.116 69.24525) (end 112.38125 76.98) (width 0.2) (layer "F.Cu") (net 5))
 (segment (start 96.77125 62.03) (end 97.37625 61.425) (width 0.2) (layer "F.Cu") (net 2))
 (segment (start 105.35625 79.45) (end 105.42625 79.52) (width 0.2) (layer "F.Cu") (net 2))
 (segment (start 97.37625 61.425) (end 102.08125 61.425) (width 0.2) (layer "F.Cu") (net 2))
 (segment (start 105.42625 79.52) (end 112.38125 79.52) (width 0.2) (layer "F.Cu") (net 2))
 (via (at 102.08125 61.425) (size 0.6) (drill 0.3) (layers "F.Cu" "B.Cu") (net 2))
 (via (at 105.35625 79.45) (size 0.6) (drill 0.3) (layers "F.Cu" "B.Cu") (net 2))
 (segment (start 102.93125 62.275) (end 102.93125 77.025) (width 0.2) (layer "B.Cu") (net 2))
 (segment (start 102.93125 77.025) (end 105.35625 79.45) (width 0.2) (layer "B.Cu") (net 2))
 (segment (start 102.08125 61.425) (end 102.93125 62.275) (width 0.2) (layer "B.Cu") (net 2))
 (segment (start 77.61125 62) (end 77.61125 74.374899) (width 0.2) (layer "F.Cu") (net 3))
 (segment (start 77.61125 74.374899) (end 83.461351 80.225) (width 0.2) (layer "F.Cu") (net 3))
 (segment (start 109.61625 82.06) (end 112.38125 82.06) (width 0.2) (layer "F.Cu") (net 3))
 (segment (start 107.78125 80.225) (end 109.61625 82.06) (width 0.2) (layer "F.Cu") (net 3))
 (segment (start 83.461351 80.225) (end 107.78125 80.225) (width 0.2) (layer "F.Cu") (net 3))
 (segment (start 112.38125 84.6) (end 102.226936 84.6) (width 0.2) (layer "F.Cu") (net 12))
 (segment (start 55.72625 61.98) (end 58.44125 61.98) (width 0.2) (layer "F.Cu") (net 12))
 (segment (start 54.65625 63.05) (end 55.72625 61.98) (width 0.2) (layer "F.Cu") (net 12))
 (segment (start 98.251936 80.625) (end 79.03125 80.625) (width 0.2) (layer "F.Cu") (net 12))
 (segment (start 79.03125 80.625) (end 65.38125 66.975) (width 0.2) (layer "F.Cu") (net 12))
 (segment (start 102.226936 84.6) (end 98.251936 80.625) (width 0.2) (layer "F.Cu") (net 12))
 (segment (start 65.38125 66.975) (end 57.95625 66.975) (width 0.2) (layer "F.Cu") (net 12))
 (via (at 54.65625 63.05) (size 0.6) (drill 0.3) (layers "F.Cu" "B.Cu") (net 12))
 (via (at 57.95625 66.975) (size 0.6) (drill 0.3) (layers "F.Cu" "B.Cu") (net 12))
 (segment (start 57.929194 66.975) (end 54.65625 63.702056) (width 0.2) (layer "B.Cu") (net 12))
 (segment (start 57.95625 66.975) (end 57.929194 66.975) (width 0.2) (layer "B.Cu") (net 12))
 (segment (start 54.65625 63.702056) (end 54.65625 63.05) (width 0.2) (layer "B.Cu") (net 12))
 (segment (start 117.226936 72.7) (end 114.18125 75.745686) (width 0.2) (layer "F.Cu") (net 4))
 (segment (start 125.10125 72.7) (end 117.226936 72.7) (width 0.2) (layer "F.Cu") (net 4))
 (segment (start 110.58125 93.52) (end 98.15625 81.095) (width 0.2) (layer "F.Cu") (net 4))
 (segment (start 114.18125 75.745686) (end 114.18125 93.52) (width 0.2) (layer "F.Cu") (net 4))
 (segment (start 98.15625 81.095) (end 77.42125 81.095) (width 0.2) (layer "F.Cu") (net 4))
 (segment (start 129.38125 76.98) (end 125.10125 72.7) (width 0.2) (layer "F.Cu") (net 4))
 (segment (start 114.18125 93.52) (end 110.58125 93.52) (width 0.2) (layer "F.Cu") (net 4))
 (segment (start 114.041935 94.225) (end 57.049652 94.225) (width 0.2) (layer "F.Cu") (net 6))
 (segment (start 57.049652 94.225) (end 43.884652 81.06) (width 0.2) (layer "F.Cu") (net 6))
 (segment (start 123.666935 84.6) (end 114.041935 94.225) (width 0.2) (layer "F.Cu") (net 6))
 (segment (start 43.884652 81.06) (end 39.29125 81.06) (width 0.2) (layer "F.Cu") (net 6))
 (segment (start 129.38125 84.6) (end 123.666935 84.6) (width 0.2) (layer "F.Cu") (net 6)))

